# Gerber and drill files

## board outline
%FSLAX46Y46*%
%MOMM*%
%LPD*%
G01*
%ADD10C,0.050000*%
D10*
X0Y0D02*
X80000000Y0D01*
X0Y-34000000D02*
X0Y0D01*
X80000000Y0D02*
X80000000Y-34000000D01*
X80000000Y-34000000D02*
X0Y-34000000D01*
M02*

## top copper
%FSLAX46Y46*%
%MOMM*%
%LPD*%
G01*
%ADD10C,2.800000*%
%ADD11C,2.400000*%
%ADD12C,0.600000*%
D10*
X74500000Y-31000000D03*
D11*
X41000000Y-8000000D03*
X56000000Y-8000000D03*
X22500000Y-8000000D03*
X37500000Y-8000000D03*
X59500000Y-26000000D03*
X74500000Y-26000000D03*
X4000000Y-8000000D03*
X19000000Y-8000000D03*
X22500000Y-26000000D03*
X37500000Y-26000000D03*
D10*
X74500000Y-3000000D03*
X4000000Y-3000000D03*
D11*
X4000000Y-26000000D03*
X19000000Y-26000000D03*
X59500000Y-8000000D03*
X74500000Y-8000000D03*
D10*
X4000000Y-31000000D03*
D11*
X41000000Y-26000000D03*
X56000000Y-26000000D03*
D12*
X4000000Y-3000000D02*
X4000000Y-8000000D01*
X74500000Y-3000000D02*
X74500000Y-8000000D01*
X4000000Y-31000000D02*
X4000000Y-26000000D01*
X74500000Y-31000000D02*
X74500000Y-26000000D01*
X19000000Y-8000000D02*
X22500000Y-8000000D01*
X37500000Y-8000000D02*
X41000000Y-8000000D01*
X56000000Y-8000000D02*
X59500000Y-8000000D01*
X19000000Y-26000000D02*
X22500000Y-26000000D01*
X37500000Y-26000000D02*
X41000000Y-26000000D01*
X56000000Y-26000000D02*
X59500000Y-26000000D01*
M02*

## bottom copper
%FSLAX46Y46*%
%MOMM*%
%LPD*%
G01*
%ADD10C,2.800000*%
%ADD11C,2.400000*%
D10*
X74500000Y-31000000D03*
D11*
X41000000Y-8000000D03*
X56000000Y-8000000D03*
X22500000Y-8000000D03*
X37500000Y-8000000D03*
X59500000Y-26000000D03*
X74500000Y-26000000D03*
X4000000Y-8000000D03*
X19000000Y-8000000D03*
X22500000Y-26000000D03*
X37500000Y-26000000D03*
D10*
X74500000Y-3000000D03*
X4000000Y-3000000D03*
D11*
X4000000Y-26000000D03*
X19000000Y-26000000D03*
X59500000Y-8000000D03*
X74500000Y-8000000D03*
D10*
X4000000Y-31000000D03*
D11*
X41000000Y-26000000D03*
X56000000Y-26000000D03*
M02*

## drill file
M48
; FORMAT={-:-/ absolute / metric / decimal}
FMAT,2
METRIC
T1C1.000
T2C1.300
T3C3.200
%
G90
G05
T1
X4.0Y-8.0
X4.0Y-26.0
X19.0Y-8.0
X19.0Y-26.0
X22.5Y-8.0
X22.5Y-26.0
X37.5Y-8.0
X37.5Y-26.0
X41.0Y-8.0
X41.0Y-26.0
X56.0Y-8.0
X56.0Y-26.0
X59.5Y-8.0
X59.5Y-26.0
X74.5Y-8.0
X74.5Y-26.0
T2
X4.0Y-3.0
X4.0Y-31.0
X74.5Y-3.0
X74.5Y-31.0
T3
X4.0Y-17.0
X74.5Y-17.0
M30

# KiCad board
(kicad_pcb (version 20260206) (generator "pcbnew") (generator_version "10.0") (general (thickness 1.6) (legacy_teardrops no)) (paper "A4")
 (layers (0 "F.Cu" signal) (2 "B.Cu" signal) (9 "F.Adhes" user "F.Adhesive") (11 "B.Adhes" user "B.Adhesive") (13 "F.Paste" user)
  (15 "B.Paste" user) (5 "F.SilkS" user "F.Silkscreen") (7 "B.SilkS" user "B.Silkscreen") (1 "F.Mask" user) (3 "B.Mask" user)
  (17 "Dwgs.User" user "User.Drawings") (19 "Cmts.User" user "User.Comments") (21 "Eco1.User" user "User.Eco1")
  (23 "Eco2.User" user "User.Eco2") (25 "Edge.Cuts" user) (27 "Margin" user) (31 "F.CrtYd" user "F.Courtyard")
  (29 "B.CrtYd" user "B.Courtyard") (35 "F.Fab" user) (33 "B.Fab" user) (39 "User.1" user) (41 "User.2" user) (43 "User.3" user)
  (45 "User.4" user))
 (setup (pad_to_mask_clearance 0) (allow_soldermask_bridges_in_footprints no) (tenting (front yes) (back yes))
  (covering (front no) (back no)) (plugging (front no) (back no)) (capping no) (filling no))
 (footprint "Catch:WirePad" (layer "F.Cu") (at 74.5 31)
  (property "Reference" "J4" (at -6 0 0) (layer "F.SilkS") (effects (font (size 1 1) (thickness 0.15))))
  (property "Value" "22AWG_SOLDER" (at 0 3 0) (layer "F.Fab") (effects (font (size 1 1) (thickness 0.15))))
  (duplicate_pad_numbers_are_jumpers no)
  (pad "1" thru_hole circle (at 0 0) (size 2.8 2.8) (drill 1.3) (layers "*.Cu" "*.Mask") (remove_unused_layers no) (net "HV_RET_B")))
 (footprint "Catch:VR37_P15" (layer "F.Cu") (at 41 8)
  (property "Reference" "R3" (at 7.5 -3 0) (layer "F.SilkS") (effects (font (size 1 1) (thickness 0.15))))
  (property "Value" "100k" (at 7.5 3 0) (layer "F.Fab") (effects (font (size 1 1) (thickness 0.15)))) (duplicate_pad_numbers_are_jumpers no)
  (pad "1" thru_hole circle (at 0 0) (size 2.4 2.4) (drill 1) (layers "*.Cu" "*.Mask") (remove_unused_layers no) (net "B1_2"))
  (pad "2" thru_hole circle (at 15 0) (size 2.4 2.4) (drill 1) (layers "*.Cu" "*.Mask") (remove_unused_layers no) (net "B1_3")))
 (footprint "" (layer "F.Cu") (at 74.5 17)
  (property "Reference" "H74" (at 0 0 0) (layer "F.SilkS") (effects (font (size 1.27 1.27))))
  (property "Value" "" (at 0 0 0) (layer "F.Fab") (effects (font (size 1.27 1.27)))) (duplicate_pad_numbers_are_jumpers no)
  (pad "" np_thru_hole circle (at 0 0) (size 3.2 3.2) (drill 3.2) (layers "*.Cu")))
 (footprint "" (layer "F.Cu") (at 4 17)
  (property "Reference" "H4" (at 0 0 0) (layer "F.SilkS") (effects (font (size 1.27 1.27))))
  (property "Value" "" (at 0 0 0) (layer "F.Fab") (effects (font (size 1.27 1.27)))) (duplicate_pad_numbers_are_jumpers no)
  (pad "" np_thru_hole circle (at 0 0) (size 3.2 3.2) (drill 3.2) (layers "*.Cu")))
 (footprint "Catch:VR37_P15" (layer "F.Cu") (at 22.5 8)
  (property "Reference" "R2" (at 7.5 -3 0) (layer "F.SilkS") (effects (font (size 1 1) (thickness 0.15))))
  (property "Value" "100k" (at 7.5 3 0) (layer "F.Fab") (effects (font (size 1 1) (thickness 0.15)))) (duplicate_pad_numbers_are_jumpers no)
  (pad "1" thru_hole circle (at 0 0) (size 2.4 2.4) (drill 1) (layers "*.Cu" "*.Mask") (remove_unused_layers no) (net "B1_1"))
  (pad "2" thru_hole circle (at 15 0) (size 2.4 2.4) (drill 1) (layers "*.Cu" "*.Mask") (remove_unused_layers no) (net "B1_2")))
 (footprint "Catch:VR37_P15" (layer "F.Cu") (at 59.5 26)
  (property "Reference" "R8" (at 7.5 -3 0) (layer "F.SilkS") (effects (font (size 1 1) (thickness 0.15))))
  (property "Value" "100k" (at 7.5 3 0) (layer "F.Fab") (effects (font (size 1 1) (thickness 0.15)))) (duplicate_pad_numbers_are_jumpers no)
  (pad "1" thru_hole circle (at 0 0) (size 2.4 2.4) (drill 1) (layers "*.Cu" "*.Mask") (remove_unused_layers no) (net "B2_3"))
  (pad "2" thru_hole circle (at 15 0) (size 2.4 2.4) (drill 1) (layers "*.Cu" "*.Mask") (remove_unused_layers no) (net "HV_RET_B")))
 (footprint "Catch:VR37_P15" (layer "F.Cu") (at 4 8)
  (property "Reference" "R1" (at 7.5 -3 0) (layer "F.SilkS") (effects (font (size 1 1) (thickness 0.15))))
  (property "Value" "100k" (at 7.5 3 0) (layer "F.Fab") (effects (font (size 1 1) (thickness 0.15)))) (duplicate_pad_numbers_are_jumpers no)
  (pad "1" thru_hole circle (at 0 0) (size 2.4 2.4) (drill 1) (layers "*.Cu" "*.Mask") (remove_unused_layers no) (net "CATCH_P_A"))
  (pad "2" thru_hole circle (at 15 0) (size 2.4 2.4) (drill 1) (layers "*.Cu" "*.Mask") (remove_unused_layers no) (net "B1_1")))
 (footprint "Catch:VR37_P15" (layer "F.Cu") (at 22.5 26)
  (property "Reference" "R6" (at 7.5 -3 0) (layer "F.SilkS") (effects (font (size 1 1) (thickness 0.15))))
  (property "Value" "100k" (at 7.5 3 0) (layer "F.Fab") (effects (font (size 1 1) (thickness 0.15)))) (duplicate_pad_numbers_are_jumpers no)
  (pad "1" thru_hole circle (at 0 0) (size 2.4 2.4) (drill 1) (layers "*.Cu" "*.Mask") (remove_unused_layers no) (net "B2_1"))
  (pad "2" thru_hole circle (at 15 0) (size 2.4 2.4) (drill 1) (layers "*.Cu" "*.Mask") (remove_unused_layers no) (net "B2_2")))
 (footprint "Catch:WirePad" (layer "F.Cu") (at 74.5 3)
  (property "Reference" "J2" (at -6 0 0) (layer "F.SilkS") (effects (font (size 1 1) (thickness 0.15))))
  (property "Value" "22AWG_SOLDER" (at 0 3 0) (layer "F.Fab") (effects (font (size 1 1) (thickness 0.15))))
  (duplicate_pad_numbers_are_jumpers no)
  (pad "1" thru_hole circle (at 0 0) (size 2.8 2.8) (drill 1.3) (layers "*.Cu" "*.Mask") (remove_unused_layers no) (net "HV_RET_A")))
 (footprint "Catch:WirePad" (layer "F.Cu") (at 4 3)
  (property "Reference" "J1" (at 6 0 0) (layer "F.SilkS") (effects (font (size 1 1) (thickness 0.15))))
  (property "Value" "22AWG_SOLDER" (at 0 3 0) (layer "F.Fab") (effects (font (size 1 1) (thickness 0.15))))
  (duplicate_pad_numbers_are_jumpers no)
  (pad "1" thru_hole circle (at 0 0) (size 2.8 2.8) (drill 1.3) (layers "*.Cu" "*.Mask") (remove_unused_layers no) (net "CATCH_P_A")))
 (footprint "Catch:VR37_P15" (layer "F.Cu") (at 4 26)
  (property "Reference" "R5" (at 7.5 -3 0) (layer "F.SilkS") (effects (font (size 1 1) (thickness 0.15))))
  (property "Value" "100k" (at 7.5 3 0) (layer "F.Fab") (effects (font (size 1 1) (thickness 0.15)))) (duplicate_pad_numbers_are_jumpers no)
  (pad "1" thru_hole circle (at 0 0) (size 2.4 2.4) (drill 1) (layers "*.Cu" "*.Mask") (remove_unused_layers no) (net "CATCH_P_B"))
  (pad "2" thru_hole circle (at 15 0) (size 2.4 2.4) (drill 1) (layers "*.Cu" "*.Mask") (remove_unused_layers no) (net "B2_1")))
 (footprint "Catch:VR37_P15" (layer "F.Cu") (at 59.5 8)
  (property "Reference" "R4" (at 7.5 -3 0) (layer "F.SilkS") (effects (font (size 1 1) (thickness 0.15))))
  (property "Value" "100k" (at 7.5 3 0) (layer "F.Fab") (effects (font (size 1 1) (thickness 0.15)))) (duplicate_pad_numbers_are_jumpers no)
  (pad "1" thru_hole circle (at 0 0) (size 2.4 2.4) (drill 1) (layers "*.Cu" "*.Mask") (remove_unused_layers no) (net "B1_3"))
  (pad "2" thru_hole circle (at 15 0) (size 2.4 2.4) (drill 1) (layers "*.Cu" "*.Mask") (remove_unused_layers no) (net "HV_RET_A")))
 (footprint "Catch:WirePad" (layer "F.Cu") (at 4 31)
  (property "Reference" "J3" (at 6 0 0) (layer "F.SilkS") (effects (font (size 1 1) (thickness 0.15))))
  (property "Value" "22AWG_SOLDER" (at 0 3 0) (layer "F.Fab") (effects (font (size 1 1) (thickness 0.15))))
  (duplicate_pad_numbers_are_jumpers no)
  (pad "1" thru_hole circle (at 0 0) (size 2.8 2.8) (drill 1.3) (layers "*.Cu" "*.Mask") (remove_unused_layers no) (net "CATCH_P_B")))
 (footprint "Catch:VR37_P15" (layer "F.Cu") (at 41 26)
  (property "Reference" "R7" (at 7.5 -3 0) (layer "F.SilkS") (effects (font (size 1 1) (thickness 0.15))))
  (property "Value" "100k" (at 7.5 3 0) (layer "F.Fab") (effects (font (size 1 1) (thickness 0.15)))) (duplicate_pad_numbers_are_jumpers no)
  (pad "1" thru_hole circle (at 0 0) (size 2.4 2.4) (drill 1) (layers "*.Cu" "*.Mask") (remove_unused_layers no) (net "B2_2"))
  (pad "2" thru_hole circle (at 15 0) (size 2.4 2.4) (drill 1) (layers "*.Cu" "*.Mask") (remove_unused_layers no) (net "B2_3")))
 (gr_line (start 0 0) (end 80 0) (stroke (width 0.05) (type default)) (layer "Edge.Cuts"))
 (gr_line (start 0 34) (end 0 0) (stroke (width 0.05) (type default)) (layer "Edge.Cuts"))
 (gr_line (start 80 0) (end 80 34) (stroke (width 0.05) (type default)) (layer "Edge.Cuts"))
 (gr_line (start 80 34) (end 0 34) (stroke (width 0.05) (type default)) (layer "Edge.Cuts"))
 (segment (start 4 3) (end 4 8) (width 0.6) (layer "F.Cu") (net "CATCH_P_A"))
 (segment (start 74.5 3) (end 74.5 8) (width 0.6) (layer "F.Cu") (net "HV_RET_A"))
 (segment (start 4 31) (end 4 26) (width 0.6) (layer "F.Cu") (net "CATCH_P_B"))
 (segment (start 74.5 31) (end 74.5 26) (width 0.6) (layer "F.Cu") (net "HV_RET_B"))
 (segment (start 19 8) (end 22.5 8) (width 0.6) (layer "F.Cu") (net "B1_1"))
 (segment (start 37.5 8) (end 41 8) (width 0.6) (layer "F.Cu") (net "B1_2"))
 (segment (start 56 8) (end 59.5 8) (width 0.6) (layer "F.Cu") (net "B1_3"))
 (segment (start 19 26) (end 22.5 26) (width 0.6) (layer "F.Cu") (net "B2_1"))
 (segment (start 37.5 26) (end 41 26) (width 0.6) (layer "F.Cu") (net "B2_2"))
 (segment (start 56 26) (end 59.5 26) (width 0.6) (layer "F.Cu") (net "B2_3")))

